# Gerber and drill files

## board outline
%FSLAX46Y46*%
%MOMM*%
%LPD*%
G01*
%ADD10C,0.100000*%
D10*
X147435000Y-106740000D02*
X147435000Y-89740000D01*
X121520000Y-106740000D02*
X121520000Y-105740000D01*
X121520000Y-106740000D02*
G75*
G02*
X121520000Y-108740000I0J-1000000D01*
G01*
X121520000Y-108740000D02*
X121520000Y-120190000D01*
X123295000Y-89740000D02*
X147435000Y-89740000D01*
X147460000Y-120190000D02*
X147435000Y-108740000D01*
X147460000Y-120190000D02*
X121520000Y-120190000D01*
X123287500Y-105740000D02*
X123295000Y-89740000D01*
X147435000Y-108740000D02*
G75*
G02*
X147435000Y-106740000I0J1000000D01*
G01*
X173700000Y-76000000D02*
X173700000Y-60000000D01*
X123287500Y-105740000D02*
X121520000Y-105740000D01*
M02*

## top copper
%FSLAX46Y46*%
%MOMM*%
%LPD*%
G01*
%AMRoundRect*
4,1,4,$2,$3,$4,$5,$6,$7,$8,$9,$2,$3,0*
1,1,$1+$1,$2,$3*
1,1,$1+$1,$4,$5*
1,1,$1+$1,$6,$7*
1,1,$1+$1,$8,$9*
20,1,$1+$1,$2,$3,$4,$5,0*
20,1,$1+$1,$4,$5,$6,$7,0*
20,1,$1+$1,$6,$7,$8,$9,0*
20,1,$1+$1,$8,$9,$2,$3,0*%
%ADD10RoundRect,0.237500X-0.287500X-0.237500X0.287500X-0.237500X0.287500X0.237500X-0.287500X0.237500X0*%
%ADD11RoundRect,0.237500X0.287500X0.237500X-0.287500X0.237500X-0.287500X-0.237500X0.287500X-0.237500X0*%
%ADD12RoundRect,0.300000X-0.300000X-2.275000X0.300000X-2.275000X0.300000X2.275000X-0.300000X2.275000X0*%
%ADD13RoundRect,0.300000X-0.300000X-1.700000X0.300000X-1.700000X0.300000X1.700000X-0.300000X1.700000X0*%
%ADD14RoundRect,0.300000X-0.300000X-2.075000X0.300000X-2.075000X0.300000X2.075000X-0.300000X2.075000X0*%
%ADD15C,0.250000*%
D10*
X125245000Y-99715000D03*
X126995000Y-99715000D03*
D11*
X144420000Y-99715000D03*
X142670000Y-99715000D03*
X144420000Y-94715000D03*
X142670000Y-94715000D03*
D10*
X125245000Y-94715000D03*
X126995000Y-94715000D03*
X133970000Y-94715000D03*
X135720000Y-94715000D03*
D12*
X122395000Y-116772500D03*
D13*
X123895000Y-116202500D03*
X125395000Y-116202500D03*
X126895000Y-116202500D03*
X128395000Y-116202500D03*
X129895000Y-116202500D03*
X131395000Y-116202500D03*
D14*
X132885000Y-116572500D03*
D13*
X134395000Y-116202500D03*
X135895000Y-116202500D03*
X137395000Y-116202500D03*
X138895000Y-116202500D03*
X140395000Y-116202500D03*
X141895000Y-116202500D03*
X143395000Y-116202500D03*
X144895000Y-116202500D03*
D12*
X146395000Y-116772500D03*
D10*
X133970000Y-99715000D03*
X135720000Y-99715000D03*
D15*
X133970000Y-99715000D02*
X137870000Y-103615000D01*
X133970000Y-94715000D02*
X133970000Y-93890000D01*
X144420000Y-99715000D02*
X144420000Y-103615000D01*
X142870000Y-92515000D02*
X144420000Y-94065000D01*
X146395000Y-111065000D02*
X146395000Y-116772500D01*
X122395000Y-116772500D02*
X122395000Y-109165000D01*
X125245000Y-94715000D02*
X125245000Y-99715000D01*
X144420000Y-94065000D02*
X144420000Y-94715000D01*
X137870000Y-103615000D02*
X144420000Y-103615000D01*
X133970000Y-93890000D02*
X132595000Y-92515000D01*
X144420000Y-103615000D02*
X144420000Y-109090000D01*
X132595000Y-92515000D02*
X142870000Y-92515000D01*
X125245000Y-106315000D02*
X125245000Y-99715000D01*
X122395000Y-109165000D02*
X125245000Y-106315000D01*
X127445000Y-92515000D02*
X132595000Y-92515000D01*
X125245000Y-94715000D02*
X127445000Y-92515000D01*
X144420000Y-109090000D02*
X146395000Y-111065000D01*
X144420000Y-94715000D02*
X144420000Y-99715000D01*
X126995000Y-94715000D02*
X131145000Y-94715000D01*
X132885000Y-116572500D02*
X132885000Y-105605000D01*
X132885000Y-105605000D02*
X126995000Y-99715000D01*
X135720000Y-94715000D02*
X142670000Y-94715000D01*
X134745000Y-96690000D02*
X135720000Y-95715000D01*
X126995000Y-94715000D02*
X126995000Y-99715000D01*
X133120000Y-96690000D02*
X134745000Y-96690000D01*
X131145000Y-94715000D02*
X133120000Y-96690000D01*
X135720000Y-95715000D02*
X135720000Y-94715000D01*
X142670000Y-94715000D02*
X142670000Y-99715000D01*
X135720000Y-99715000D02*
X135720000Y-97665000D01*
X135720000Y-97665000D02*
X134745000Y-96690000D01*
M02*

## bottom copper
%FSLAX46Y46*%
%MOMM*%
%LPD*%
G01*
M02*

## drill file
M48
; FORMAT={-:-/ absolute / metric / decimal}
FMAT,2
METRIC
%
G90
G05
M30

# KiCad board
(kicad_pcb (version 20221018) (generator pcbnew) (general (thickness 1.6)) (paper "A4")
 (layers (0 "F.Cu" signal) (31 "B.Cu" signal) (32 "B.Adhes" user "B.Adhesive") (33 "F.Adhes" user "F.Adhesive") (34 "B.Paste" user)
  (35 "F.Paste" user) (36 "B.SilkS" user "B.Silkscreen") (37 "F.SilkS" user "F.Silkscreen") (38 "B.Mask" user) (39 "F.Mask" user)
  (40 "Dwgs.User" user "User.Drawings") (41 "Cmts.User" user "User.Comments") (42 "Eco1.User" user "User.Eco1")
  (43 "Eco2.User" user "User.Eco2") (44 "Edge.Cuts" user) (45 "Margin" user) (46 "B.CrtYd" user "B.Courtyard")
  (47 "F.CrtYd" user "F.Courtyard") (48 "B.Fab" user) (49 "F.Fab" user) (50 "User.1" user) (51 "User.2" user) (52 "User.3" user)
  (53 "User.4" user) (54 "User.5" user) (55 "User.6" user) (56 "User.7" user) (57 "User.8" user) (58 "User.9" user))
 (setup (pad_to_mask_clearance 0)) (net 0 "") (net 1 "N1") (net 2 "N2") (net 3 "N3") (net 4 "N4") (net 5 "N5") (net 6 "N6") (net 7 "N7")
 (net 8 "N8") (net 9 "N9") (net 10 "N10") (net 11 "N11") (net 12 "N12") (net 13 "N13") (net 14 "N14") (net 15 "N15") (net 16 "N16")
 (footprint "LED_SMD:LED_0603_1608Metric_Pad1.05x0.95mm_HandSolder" (layer "F.Cu") (at 126.12 99.715)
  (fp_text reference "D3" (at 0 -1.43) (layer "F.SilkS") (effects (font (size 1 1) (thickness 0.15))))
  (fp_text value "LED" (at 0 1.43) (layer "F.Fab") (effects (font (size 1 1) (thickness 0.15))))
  (pad "1" smd roundrect (at -0.875 0) (size 1.05 0.95) (layers "F.Cu" "F.Paste" "F.Mask") (roundrect_rratio 0.25) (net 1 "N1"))
  (pad "2" smd roundrect (at 0.875 0) (size 1.05 0.95) (layers "F.Cu" "F.Paste" "F.Mask") (roundrect_rratio 0.25) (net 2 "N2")))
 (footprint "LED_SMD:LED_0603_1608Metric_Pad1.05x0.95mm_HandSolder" (layer "F.Cu") (at 143.545 99.715 180)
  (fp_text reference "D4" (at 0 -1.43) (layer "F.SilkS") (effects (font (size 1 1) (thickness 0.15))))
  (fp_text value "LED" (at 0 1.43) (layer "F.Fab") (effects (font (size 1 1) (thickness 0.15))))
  (pad "1" smd roundrect (at -0.875 0 180) (size 1.05 0.95) (layers "F.Cu" "F.Paste" "F.Mask") (roundrect_rratio 0.25) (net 1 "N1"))
  (pad "2" smd roundrect (at 0.875 0 180) (size 1.05 0.95) (layers "F.Cu" "F.Paste" "F.Mask") (roundrect_rratio 0.25) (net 2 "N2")))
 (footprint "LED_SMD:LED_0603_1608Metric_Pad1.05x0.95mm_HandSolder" (layer "F.Cu") (at 143.545 94.715 180)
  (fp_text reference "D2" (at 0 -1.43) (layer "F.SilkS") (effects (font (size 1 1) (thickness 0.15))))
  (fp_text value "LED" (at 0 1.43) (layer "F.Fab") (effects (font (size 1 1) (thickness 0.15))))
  (pad "1" smd roundrect (at -0.875 0 180) (size 1.05 0.95) (layers "F.Cu" "F.Paste" "F.Mask") (roundrect_rratio 0.25) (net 1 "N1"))
  (pad "2" smd roundrect (at 0.875 0 180) (size 1.05 0.95) (layers "F.Cu" "F.Paste" "F.Mask") (roundrect_rratio 0.25) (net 2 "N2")))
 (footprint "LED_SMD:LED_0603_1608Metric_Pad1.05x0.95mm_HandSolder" (layer "F.Cu") (at 126.12 94.715)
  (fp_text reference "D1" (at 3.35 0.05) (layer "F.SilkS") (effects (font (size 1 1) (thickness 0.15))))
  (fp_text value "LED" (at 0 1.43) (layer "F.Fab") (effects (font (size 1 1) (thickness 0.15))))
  (pad "1" smd roundrect (at -0.875 0) (size 1.05 0.95) (layers "F.Cu" "F.Paste" "F.Mask") (roundrect_rratio 0.25) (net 1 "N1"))
  (pad "2" smd roundrect (at 0.875 0) (size 1.05 0.95) (layers "F.Cu" "F.Paste" "F.Mask") (roundrect_rratio 0.25) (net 2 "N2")))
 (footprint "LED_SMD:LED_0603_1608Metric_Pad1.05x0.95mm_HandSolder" (layer "F.Cu") (at 134.845 94.715)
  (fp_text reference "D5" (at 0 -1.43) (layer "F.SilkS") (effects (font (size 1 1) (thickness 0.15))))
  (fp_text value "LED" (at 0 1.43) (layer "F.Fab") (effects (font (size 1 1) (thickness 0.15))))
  (pad "1" smd roundrect (at -0.875 0) (size 1.05 0.95) (layers "F.Cu" "F.Paste" "F.Mask") (roundrect_rratio 0.25) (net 1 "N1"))
  (pad "2" smd roundrect (at 0.875 0) (size 1.05 0.95) (layers "F.Cu" "F.Paste" "F.Mask") (roundrect_rratio 0.25) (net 2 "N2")))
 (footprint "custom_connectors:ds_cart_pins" (layer "F.Cu") (at 134.405 116.2125)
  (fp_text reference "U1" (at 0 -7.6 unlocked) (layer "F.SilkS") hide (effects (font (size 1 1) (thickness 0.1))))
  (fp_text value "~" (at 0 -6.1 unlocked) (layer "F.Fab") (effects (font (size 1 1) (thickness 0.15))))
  (pad "1" smd roundrect (at -12.01 0.56) (size 1.2 5.15) (layers "F.Cu" "F.Paste" "F.Mask") (roundrect_rratio 0.25) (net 1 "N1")
   (thermal_bridge_angle 45))
  (pad "2" smd roundrect (at -10.51 -0.01) (size 1.2 4) (layers "F.Cu" "F.Paste" "F.Mask") (roundrect_rratio 0.25) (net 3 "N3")
   (thermal_bridge_angle 45))
  (pad "3" smd roundrect (at -9.01 -0.01) (size 1.2 4) (layers "F.Cu" "F.Paste" "F.Mask") (roundrect_rratio 0.25) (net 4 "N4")
   (thermal_bridge_angle 45))
  (pad "4" smd roundrect (at -7.51 -0.01) (size 1.2 4) (layers "F.Cu" "F.Paste" "F.Mask") (roundrect_rratio 0.25) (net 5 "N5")
   (thermal_bridge_angle 45))
  (pad "5" smd roundrect (at -6.01 -0.01) (size 1.2 4) (layers "F.Cu" "F.Paste" "F.Mask") (roundrect_rratio 0.25) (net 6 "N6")
   (thermal_bridge_angle 45))
  (pad "6" smd roundrect (at -4.51 -0.01) (size 1.2 4) (layers "F.Cu" "F.Paste" "F.Mask") (roundrect_rratio 0.25) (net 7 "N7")
   (thermal_bridge_angle 45))
  (pad "7" smd roundrect (at -3.01 -0.01) (size 1.2 4) (layers "F.Cu" "F.Paste" "F.Mask") (roundrect_rratio 0.25) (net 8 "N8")
   (thermal_bridge_angle 45))
  (pad "8" smd roundrect (at -1.52 0.36) (size 1.2 4.75) (layers "F.Cu" "F.Paste" "F.Mask") (roundrect_rratio 0.25) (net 2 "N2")
   (thermal_bridge_angle 45))
  (pad "9" smd roundrect (at -0.01 -0.01) (size 1.2 4) (layers "F.Cu" "F.Paste" "F.Mask") (roundrect_rratio 0.25) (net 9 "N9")
   (thermal_bridge_angle 45))
  (pad "10" smd roundrect (at 1.49 -0.01) (size 1.2 4) (layers "F.Cu" "F.Paste" "F.Mask") (roundrect_rratio 0.25) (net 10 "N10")
   (thermal_bridge_angle 45))
  (pad "11" smd roundrect (at 2.99 -0.01) (size 1.2 4) (layers "F.Cu" "F.Paste" "F.Mask") (roundrect_rratio 0.25) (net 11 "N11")
   (thermal_bridge_angle 45))
  (pad "12" smd roundrect (at 4.49 -0.01) (size 1.2 4) (layers "F.Cu" "F.Paste" "F.Mask") (roundrect_rratio 0.25) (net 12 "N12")
   (thermal_bridge_angle 45))
  (pad "13" smd roundrect (at 5.99 -0.01) (size 1.2 4) (layers "F.Cu" "F.Paste" "F.Mask") (roundrect_rratio 0.25) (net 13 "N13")
   (thermal_bridge_angle 45))
  (pad "14" smd roundrect (at 7.49 -0.01) (size 1.2 4) (layers "F.Cu" "F.Paste" "F.Mask") (roundrect_rratio 0.25) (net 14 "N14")
   (thermal_bridge_angle 45))
  (pad "15" smd roundrect (at 8.99 -0.01) (size 1.2 4) (layers "F.Cu" "F.Paste" "F.Mask") (roundrect_rratio 0.25) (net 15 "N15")
   (thermal_bridge_angle 45))
  (pad "16" smd roundrect (at 10.49 -0.01) (size 1.2 4) (layers "F.Cu" "F.Paste" "F.Mask") (roundrect_rratio 0.25) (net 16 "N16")
   (thermal_bridge_angle 45))
  (pad "17" smd roundrect (at 11.99 0.56) (size 1.2 5.15) (layers "F.Cu" "F.Paste" "F.Mask") (roundrect_rratio 0.25) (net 1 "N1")
   (thermal_bridge_angle 45)))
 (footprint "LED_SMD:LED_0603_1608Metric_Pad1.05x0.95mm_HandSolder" (layer "F.Cu") (at 134.845 99.715)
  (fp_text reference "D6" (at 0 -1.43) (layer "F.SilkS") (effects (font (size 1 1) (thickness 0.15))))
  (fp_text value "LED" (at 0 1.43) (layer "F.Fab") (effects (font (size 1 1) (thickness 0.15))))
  (pad "1" smd roundrect (at -0.875 0) (size 1.05 0.95) (layers "F.Cu" "F.Paste" "F.Mask") (roundrect_rratio 0.25) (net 1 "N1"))
  (pad "2" smd roundrect (at 0.875 0) (size 1.05 0.95) (layers "F.Cu" "F.Paste" "F.Mask") (roundrect_rratio 0.25) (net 2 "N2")))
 (gr_line (start 147.435 106.74) (end 147.435 89.74) (stroke (width 0.1) (type default)) (layer "Edge.Cuts"))
 (gr_line (start 121.52 106.74) (end 121.52 105.74) (stroke (width 0.1) (type default)) (layer "Edge.Cuts"))
 (gr_arc (start 121.52 106.74) (mid 122.52 107.74) (end 121.52 108.74) (stroke (width 0.1) (type default)) (layer "Edge.Cuts"))
 (gr_line (start 121.52 108.74) (end 121.52 120.19) (stroke (width 0.1) (type default)) (layer "Edge.Cuts"))
 (gr_line (start 123.295 89.74) (end 147.435 89.74) (stroke (width 0.1) (type default)) (layer "Edge.Cuts"))
 (gr_line (start 147.46 120.19) (end 147.435 108.74) (stroke (width 0.1) (type default)) (layer "Edge.Cuts"))
 (gr_line (start 147.46 120.19) (end 121.52 120.19) (stroke (width 0.1) (type default)) (layer "Edge.Cuts"))
 (gr_line (start 123.2875 105.74) (end 123.295 89.74) (stroke (width 0.1) (type default)) (layer "Edge.Cuts"))
 (gr_arc (start 147.435 108.74) (mid 146.435 107.74) (end 147.435 106.74) (stroke (width 0.1) (type default)) (layer "Edge.Cuts"))
 (gr_line locked (start 173.7 76) (end 173.7 60) (stroke (width 0.1) (type default)) (layer "Edge.Cuts"))
 (gr_line (start 123.2875 105.74) (end 121.52 105.74) (stroke (width 0.1) (type default)) (layer "Edge.Cuts"))
 (segment (start 133.97 99.715) (end 137.87 103.615) (width 0.25) (layer "F.Cu") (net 1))
 (segment (start 133.97 94.715) (end 133.97 93.89) (width 0.25) (layer "F.Cu") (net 1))
 (segment (start 144.42 99.715) (end 144.42 103.615) (width 0.25) (layer "F.Cu") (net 1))
 (segment (start 142.87 92.515) (end 144.42 94.065) (width 0.25) (layer "F.Cu") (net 1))
 (segment (start 146.395 111.065) (end 146.395 116.7725) (width 0.25) (layer "F.Cu") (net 1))
 (segment (start 122.395 116.7725) (end 122.395 109.165) (width 0.25) (layer "F.Cu") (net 1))
 (segment (start 125.245 94.715) (end 125.245 99.715) (width 0.25) (layer "F.Cu") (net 1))
 (segment (start 144.42 94.065) (end 144.42 94.715) (width 0.25) (layer "F.Cu") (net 1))
 (segment (start 137.87 103.615) (end 144.42 103.615) (width 0.25) (layer "F.Cu") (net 1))
 (segment (start 133.97 93.89) (end 132.595 92.515) (width 0.25) (layer "F.Cu") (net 1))
 (segment (start 144.42 103.615) (end 144.42 109.09) (width 0.25) (layer "F.Cu") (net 1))
 (segment (start 132.595 92.515) (end 142.87 92.515) (width 0.25) (layer "F.Cu") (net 1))
 (segment (start 125.245 106.315) (end 125.245 99.715) (width 0.25) (layer "F.Cu") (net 1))
 (segment (start 122.395 109.165) (end 125.245 106.315) (width 0.25) (layer "F.Cu") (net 1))
 (segment (start 127.445 92.515) (end 132.595 92.515) (width 0.25) (layer "F.Cu") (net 1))
 (segment (start 125.245 94.715) (end 127.445 92.515) (width 0.25) (layer "F.Cu") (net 1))
 (segment (start 144.42 109.09) (end 146.395 111.065) (width 0.25) (layer "F.Cu") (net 1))
 (segment (start 144.42 94.715) (end 144.42 99.715) (width 0.25) (layer "F.Cu") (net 1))
 (segment (start 126.995 94.715) (end 131.145 94.715) (width 0.25) (layer "F.Cu") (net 2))
 (segment (start 132.885 116.5725) (end 132.885 105.605) (width 0.25) (layer "F.Cu") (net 2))
 (segment (start 132.885 105.605) (end 126.995 99.715) (width 0.25) (layer "F.Cu") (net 2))
 (segment (start 135.72 94.715) (end 142.67 94.715) (width 0.25) (layer "F.Cu") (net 2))
 (segment (start 134.745 96.69) (end 135.72 95.715) (width 0.25) (layer "F.Cu") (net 2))
 (segment (start 126.995 94.715) (end 126.995 99.715) (width 0.25) (layer "F.Cu") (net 2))
 (segment (start 133.12 96.69) (end 134.745 96.69) (width 0.25) (layer "F.Cu") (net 2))
 (segment (start 131.145 94.715) (end 133.12 96.69) (width 0.25) (layer "F.Cu") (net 2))
 (segment (start 135.72 95.715) (end 135.72 94.715) (width 0.25) (layer "F.Cu") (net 2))
 (segment (start 142.67 94.715) (end 142.67 99.715) (width 0.25) (layer "F.Cu") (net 2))
 (segment (start 135.72 99.715) (end 135.72 97.665) (width 0.25) (layer "F.Cu") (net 2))
 (segment (start 135.72 97.665) (end 134.745 96.69) (width 0.25) (layer "F.Cu") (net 2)))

